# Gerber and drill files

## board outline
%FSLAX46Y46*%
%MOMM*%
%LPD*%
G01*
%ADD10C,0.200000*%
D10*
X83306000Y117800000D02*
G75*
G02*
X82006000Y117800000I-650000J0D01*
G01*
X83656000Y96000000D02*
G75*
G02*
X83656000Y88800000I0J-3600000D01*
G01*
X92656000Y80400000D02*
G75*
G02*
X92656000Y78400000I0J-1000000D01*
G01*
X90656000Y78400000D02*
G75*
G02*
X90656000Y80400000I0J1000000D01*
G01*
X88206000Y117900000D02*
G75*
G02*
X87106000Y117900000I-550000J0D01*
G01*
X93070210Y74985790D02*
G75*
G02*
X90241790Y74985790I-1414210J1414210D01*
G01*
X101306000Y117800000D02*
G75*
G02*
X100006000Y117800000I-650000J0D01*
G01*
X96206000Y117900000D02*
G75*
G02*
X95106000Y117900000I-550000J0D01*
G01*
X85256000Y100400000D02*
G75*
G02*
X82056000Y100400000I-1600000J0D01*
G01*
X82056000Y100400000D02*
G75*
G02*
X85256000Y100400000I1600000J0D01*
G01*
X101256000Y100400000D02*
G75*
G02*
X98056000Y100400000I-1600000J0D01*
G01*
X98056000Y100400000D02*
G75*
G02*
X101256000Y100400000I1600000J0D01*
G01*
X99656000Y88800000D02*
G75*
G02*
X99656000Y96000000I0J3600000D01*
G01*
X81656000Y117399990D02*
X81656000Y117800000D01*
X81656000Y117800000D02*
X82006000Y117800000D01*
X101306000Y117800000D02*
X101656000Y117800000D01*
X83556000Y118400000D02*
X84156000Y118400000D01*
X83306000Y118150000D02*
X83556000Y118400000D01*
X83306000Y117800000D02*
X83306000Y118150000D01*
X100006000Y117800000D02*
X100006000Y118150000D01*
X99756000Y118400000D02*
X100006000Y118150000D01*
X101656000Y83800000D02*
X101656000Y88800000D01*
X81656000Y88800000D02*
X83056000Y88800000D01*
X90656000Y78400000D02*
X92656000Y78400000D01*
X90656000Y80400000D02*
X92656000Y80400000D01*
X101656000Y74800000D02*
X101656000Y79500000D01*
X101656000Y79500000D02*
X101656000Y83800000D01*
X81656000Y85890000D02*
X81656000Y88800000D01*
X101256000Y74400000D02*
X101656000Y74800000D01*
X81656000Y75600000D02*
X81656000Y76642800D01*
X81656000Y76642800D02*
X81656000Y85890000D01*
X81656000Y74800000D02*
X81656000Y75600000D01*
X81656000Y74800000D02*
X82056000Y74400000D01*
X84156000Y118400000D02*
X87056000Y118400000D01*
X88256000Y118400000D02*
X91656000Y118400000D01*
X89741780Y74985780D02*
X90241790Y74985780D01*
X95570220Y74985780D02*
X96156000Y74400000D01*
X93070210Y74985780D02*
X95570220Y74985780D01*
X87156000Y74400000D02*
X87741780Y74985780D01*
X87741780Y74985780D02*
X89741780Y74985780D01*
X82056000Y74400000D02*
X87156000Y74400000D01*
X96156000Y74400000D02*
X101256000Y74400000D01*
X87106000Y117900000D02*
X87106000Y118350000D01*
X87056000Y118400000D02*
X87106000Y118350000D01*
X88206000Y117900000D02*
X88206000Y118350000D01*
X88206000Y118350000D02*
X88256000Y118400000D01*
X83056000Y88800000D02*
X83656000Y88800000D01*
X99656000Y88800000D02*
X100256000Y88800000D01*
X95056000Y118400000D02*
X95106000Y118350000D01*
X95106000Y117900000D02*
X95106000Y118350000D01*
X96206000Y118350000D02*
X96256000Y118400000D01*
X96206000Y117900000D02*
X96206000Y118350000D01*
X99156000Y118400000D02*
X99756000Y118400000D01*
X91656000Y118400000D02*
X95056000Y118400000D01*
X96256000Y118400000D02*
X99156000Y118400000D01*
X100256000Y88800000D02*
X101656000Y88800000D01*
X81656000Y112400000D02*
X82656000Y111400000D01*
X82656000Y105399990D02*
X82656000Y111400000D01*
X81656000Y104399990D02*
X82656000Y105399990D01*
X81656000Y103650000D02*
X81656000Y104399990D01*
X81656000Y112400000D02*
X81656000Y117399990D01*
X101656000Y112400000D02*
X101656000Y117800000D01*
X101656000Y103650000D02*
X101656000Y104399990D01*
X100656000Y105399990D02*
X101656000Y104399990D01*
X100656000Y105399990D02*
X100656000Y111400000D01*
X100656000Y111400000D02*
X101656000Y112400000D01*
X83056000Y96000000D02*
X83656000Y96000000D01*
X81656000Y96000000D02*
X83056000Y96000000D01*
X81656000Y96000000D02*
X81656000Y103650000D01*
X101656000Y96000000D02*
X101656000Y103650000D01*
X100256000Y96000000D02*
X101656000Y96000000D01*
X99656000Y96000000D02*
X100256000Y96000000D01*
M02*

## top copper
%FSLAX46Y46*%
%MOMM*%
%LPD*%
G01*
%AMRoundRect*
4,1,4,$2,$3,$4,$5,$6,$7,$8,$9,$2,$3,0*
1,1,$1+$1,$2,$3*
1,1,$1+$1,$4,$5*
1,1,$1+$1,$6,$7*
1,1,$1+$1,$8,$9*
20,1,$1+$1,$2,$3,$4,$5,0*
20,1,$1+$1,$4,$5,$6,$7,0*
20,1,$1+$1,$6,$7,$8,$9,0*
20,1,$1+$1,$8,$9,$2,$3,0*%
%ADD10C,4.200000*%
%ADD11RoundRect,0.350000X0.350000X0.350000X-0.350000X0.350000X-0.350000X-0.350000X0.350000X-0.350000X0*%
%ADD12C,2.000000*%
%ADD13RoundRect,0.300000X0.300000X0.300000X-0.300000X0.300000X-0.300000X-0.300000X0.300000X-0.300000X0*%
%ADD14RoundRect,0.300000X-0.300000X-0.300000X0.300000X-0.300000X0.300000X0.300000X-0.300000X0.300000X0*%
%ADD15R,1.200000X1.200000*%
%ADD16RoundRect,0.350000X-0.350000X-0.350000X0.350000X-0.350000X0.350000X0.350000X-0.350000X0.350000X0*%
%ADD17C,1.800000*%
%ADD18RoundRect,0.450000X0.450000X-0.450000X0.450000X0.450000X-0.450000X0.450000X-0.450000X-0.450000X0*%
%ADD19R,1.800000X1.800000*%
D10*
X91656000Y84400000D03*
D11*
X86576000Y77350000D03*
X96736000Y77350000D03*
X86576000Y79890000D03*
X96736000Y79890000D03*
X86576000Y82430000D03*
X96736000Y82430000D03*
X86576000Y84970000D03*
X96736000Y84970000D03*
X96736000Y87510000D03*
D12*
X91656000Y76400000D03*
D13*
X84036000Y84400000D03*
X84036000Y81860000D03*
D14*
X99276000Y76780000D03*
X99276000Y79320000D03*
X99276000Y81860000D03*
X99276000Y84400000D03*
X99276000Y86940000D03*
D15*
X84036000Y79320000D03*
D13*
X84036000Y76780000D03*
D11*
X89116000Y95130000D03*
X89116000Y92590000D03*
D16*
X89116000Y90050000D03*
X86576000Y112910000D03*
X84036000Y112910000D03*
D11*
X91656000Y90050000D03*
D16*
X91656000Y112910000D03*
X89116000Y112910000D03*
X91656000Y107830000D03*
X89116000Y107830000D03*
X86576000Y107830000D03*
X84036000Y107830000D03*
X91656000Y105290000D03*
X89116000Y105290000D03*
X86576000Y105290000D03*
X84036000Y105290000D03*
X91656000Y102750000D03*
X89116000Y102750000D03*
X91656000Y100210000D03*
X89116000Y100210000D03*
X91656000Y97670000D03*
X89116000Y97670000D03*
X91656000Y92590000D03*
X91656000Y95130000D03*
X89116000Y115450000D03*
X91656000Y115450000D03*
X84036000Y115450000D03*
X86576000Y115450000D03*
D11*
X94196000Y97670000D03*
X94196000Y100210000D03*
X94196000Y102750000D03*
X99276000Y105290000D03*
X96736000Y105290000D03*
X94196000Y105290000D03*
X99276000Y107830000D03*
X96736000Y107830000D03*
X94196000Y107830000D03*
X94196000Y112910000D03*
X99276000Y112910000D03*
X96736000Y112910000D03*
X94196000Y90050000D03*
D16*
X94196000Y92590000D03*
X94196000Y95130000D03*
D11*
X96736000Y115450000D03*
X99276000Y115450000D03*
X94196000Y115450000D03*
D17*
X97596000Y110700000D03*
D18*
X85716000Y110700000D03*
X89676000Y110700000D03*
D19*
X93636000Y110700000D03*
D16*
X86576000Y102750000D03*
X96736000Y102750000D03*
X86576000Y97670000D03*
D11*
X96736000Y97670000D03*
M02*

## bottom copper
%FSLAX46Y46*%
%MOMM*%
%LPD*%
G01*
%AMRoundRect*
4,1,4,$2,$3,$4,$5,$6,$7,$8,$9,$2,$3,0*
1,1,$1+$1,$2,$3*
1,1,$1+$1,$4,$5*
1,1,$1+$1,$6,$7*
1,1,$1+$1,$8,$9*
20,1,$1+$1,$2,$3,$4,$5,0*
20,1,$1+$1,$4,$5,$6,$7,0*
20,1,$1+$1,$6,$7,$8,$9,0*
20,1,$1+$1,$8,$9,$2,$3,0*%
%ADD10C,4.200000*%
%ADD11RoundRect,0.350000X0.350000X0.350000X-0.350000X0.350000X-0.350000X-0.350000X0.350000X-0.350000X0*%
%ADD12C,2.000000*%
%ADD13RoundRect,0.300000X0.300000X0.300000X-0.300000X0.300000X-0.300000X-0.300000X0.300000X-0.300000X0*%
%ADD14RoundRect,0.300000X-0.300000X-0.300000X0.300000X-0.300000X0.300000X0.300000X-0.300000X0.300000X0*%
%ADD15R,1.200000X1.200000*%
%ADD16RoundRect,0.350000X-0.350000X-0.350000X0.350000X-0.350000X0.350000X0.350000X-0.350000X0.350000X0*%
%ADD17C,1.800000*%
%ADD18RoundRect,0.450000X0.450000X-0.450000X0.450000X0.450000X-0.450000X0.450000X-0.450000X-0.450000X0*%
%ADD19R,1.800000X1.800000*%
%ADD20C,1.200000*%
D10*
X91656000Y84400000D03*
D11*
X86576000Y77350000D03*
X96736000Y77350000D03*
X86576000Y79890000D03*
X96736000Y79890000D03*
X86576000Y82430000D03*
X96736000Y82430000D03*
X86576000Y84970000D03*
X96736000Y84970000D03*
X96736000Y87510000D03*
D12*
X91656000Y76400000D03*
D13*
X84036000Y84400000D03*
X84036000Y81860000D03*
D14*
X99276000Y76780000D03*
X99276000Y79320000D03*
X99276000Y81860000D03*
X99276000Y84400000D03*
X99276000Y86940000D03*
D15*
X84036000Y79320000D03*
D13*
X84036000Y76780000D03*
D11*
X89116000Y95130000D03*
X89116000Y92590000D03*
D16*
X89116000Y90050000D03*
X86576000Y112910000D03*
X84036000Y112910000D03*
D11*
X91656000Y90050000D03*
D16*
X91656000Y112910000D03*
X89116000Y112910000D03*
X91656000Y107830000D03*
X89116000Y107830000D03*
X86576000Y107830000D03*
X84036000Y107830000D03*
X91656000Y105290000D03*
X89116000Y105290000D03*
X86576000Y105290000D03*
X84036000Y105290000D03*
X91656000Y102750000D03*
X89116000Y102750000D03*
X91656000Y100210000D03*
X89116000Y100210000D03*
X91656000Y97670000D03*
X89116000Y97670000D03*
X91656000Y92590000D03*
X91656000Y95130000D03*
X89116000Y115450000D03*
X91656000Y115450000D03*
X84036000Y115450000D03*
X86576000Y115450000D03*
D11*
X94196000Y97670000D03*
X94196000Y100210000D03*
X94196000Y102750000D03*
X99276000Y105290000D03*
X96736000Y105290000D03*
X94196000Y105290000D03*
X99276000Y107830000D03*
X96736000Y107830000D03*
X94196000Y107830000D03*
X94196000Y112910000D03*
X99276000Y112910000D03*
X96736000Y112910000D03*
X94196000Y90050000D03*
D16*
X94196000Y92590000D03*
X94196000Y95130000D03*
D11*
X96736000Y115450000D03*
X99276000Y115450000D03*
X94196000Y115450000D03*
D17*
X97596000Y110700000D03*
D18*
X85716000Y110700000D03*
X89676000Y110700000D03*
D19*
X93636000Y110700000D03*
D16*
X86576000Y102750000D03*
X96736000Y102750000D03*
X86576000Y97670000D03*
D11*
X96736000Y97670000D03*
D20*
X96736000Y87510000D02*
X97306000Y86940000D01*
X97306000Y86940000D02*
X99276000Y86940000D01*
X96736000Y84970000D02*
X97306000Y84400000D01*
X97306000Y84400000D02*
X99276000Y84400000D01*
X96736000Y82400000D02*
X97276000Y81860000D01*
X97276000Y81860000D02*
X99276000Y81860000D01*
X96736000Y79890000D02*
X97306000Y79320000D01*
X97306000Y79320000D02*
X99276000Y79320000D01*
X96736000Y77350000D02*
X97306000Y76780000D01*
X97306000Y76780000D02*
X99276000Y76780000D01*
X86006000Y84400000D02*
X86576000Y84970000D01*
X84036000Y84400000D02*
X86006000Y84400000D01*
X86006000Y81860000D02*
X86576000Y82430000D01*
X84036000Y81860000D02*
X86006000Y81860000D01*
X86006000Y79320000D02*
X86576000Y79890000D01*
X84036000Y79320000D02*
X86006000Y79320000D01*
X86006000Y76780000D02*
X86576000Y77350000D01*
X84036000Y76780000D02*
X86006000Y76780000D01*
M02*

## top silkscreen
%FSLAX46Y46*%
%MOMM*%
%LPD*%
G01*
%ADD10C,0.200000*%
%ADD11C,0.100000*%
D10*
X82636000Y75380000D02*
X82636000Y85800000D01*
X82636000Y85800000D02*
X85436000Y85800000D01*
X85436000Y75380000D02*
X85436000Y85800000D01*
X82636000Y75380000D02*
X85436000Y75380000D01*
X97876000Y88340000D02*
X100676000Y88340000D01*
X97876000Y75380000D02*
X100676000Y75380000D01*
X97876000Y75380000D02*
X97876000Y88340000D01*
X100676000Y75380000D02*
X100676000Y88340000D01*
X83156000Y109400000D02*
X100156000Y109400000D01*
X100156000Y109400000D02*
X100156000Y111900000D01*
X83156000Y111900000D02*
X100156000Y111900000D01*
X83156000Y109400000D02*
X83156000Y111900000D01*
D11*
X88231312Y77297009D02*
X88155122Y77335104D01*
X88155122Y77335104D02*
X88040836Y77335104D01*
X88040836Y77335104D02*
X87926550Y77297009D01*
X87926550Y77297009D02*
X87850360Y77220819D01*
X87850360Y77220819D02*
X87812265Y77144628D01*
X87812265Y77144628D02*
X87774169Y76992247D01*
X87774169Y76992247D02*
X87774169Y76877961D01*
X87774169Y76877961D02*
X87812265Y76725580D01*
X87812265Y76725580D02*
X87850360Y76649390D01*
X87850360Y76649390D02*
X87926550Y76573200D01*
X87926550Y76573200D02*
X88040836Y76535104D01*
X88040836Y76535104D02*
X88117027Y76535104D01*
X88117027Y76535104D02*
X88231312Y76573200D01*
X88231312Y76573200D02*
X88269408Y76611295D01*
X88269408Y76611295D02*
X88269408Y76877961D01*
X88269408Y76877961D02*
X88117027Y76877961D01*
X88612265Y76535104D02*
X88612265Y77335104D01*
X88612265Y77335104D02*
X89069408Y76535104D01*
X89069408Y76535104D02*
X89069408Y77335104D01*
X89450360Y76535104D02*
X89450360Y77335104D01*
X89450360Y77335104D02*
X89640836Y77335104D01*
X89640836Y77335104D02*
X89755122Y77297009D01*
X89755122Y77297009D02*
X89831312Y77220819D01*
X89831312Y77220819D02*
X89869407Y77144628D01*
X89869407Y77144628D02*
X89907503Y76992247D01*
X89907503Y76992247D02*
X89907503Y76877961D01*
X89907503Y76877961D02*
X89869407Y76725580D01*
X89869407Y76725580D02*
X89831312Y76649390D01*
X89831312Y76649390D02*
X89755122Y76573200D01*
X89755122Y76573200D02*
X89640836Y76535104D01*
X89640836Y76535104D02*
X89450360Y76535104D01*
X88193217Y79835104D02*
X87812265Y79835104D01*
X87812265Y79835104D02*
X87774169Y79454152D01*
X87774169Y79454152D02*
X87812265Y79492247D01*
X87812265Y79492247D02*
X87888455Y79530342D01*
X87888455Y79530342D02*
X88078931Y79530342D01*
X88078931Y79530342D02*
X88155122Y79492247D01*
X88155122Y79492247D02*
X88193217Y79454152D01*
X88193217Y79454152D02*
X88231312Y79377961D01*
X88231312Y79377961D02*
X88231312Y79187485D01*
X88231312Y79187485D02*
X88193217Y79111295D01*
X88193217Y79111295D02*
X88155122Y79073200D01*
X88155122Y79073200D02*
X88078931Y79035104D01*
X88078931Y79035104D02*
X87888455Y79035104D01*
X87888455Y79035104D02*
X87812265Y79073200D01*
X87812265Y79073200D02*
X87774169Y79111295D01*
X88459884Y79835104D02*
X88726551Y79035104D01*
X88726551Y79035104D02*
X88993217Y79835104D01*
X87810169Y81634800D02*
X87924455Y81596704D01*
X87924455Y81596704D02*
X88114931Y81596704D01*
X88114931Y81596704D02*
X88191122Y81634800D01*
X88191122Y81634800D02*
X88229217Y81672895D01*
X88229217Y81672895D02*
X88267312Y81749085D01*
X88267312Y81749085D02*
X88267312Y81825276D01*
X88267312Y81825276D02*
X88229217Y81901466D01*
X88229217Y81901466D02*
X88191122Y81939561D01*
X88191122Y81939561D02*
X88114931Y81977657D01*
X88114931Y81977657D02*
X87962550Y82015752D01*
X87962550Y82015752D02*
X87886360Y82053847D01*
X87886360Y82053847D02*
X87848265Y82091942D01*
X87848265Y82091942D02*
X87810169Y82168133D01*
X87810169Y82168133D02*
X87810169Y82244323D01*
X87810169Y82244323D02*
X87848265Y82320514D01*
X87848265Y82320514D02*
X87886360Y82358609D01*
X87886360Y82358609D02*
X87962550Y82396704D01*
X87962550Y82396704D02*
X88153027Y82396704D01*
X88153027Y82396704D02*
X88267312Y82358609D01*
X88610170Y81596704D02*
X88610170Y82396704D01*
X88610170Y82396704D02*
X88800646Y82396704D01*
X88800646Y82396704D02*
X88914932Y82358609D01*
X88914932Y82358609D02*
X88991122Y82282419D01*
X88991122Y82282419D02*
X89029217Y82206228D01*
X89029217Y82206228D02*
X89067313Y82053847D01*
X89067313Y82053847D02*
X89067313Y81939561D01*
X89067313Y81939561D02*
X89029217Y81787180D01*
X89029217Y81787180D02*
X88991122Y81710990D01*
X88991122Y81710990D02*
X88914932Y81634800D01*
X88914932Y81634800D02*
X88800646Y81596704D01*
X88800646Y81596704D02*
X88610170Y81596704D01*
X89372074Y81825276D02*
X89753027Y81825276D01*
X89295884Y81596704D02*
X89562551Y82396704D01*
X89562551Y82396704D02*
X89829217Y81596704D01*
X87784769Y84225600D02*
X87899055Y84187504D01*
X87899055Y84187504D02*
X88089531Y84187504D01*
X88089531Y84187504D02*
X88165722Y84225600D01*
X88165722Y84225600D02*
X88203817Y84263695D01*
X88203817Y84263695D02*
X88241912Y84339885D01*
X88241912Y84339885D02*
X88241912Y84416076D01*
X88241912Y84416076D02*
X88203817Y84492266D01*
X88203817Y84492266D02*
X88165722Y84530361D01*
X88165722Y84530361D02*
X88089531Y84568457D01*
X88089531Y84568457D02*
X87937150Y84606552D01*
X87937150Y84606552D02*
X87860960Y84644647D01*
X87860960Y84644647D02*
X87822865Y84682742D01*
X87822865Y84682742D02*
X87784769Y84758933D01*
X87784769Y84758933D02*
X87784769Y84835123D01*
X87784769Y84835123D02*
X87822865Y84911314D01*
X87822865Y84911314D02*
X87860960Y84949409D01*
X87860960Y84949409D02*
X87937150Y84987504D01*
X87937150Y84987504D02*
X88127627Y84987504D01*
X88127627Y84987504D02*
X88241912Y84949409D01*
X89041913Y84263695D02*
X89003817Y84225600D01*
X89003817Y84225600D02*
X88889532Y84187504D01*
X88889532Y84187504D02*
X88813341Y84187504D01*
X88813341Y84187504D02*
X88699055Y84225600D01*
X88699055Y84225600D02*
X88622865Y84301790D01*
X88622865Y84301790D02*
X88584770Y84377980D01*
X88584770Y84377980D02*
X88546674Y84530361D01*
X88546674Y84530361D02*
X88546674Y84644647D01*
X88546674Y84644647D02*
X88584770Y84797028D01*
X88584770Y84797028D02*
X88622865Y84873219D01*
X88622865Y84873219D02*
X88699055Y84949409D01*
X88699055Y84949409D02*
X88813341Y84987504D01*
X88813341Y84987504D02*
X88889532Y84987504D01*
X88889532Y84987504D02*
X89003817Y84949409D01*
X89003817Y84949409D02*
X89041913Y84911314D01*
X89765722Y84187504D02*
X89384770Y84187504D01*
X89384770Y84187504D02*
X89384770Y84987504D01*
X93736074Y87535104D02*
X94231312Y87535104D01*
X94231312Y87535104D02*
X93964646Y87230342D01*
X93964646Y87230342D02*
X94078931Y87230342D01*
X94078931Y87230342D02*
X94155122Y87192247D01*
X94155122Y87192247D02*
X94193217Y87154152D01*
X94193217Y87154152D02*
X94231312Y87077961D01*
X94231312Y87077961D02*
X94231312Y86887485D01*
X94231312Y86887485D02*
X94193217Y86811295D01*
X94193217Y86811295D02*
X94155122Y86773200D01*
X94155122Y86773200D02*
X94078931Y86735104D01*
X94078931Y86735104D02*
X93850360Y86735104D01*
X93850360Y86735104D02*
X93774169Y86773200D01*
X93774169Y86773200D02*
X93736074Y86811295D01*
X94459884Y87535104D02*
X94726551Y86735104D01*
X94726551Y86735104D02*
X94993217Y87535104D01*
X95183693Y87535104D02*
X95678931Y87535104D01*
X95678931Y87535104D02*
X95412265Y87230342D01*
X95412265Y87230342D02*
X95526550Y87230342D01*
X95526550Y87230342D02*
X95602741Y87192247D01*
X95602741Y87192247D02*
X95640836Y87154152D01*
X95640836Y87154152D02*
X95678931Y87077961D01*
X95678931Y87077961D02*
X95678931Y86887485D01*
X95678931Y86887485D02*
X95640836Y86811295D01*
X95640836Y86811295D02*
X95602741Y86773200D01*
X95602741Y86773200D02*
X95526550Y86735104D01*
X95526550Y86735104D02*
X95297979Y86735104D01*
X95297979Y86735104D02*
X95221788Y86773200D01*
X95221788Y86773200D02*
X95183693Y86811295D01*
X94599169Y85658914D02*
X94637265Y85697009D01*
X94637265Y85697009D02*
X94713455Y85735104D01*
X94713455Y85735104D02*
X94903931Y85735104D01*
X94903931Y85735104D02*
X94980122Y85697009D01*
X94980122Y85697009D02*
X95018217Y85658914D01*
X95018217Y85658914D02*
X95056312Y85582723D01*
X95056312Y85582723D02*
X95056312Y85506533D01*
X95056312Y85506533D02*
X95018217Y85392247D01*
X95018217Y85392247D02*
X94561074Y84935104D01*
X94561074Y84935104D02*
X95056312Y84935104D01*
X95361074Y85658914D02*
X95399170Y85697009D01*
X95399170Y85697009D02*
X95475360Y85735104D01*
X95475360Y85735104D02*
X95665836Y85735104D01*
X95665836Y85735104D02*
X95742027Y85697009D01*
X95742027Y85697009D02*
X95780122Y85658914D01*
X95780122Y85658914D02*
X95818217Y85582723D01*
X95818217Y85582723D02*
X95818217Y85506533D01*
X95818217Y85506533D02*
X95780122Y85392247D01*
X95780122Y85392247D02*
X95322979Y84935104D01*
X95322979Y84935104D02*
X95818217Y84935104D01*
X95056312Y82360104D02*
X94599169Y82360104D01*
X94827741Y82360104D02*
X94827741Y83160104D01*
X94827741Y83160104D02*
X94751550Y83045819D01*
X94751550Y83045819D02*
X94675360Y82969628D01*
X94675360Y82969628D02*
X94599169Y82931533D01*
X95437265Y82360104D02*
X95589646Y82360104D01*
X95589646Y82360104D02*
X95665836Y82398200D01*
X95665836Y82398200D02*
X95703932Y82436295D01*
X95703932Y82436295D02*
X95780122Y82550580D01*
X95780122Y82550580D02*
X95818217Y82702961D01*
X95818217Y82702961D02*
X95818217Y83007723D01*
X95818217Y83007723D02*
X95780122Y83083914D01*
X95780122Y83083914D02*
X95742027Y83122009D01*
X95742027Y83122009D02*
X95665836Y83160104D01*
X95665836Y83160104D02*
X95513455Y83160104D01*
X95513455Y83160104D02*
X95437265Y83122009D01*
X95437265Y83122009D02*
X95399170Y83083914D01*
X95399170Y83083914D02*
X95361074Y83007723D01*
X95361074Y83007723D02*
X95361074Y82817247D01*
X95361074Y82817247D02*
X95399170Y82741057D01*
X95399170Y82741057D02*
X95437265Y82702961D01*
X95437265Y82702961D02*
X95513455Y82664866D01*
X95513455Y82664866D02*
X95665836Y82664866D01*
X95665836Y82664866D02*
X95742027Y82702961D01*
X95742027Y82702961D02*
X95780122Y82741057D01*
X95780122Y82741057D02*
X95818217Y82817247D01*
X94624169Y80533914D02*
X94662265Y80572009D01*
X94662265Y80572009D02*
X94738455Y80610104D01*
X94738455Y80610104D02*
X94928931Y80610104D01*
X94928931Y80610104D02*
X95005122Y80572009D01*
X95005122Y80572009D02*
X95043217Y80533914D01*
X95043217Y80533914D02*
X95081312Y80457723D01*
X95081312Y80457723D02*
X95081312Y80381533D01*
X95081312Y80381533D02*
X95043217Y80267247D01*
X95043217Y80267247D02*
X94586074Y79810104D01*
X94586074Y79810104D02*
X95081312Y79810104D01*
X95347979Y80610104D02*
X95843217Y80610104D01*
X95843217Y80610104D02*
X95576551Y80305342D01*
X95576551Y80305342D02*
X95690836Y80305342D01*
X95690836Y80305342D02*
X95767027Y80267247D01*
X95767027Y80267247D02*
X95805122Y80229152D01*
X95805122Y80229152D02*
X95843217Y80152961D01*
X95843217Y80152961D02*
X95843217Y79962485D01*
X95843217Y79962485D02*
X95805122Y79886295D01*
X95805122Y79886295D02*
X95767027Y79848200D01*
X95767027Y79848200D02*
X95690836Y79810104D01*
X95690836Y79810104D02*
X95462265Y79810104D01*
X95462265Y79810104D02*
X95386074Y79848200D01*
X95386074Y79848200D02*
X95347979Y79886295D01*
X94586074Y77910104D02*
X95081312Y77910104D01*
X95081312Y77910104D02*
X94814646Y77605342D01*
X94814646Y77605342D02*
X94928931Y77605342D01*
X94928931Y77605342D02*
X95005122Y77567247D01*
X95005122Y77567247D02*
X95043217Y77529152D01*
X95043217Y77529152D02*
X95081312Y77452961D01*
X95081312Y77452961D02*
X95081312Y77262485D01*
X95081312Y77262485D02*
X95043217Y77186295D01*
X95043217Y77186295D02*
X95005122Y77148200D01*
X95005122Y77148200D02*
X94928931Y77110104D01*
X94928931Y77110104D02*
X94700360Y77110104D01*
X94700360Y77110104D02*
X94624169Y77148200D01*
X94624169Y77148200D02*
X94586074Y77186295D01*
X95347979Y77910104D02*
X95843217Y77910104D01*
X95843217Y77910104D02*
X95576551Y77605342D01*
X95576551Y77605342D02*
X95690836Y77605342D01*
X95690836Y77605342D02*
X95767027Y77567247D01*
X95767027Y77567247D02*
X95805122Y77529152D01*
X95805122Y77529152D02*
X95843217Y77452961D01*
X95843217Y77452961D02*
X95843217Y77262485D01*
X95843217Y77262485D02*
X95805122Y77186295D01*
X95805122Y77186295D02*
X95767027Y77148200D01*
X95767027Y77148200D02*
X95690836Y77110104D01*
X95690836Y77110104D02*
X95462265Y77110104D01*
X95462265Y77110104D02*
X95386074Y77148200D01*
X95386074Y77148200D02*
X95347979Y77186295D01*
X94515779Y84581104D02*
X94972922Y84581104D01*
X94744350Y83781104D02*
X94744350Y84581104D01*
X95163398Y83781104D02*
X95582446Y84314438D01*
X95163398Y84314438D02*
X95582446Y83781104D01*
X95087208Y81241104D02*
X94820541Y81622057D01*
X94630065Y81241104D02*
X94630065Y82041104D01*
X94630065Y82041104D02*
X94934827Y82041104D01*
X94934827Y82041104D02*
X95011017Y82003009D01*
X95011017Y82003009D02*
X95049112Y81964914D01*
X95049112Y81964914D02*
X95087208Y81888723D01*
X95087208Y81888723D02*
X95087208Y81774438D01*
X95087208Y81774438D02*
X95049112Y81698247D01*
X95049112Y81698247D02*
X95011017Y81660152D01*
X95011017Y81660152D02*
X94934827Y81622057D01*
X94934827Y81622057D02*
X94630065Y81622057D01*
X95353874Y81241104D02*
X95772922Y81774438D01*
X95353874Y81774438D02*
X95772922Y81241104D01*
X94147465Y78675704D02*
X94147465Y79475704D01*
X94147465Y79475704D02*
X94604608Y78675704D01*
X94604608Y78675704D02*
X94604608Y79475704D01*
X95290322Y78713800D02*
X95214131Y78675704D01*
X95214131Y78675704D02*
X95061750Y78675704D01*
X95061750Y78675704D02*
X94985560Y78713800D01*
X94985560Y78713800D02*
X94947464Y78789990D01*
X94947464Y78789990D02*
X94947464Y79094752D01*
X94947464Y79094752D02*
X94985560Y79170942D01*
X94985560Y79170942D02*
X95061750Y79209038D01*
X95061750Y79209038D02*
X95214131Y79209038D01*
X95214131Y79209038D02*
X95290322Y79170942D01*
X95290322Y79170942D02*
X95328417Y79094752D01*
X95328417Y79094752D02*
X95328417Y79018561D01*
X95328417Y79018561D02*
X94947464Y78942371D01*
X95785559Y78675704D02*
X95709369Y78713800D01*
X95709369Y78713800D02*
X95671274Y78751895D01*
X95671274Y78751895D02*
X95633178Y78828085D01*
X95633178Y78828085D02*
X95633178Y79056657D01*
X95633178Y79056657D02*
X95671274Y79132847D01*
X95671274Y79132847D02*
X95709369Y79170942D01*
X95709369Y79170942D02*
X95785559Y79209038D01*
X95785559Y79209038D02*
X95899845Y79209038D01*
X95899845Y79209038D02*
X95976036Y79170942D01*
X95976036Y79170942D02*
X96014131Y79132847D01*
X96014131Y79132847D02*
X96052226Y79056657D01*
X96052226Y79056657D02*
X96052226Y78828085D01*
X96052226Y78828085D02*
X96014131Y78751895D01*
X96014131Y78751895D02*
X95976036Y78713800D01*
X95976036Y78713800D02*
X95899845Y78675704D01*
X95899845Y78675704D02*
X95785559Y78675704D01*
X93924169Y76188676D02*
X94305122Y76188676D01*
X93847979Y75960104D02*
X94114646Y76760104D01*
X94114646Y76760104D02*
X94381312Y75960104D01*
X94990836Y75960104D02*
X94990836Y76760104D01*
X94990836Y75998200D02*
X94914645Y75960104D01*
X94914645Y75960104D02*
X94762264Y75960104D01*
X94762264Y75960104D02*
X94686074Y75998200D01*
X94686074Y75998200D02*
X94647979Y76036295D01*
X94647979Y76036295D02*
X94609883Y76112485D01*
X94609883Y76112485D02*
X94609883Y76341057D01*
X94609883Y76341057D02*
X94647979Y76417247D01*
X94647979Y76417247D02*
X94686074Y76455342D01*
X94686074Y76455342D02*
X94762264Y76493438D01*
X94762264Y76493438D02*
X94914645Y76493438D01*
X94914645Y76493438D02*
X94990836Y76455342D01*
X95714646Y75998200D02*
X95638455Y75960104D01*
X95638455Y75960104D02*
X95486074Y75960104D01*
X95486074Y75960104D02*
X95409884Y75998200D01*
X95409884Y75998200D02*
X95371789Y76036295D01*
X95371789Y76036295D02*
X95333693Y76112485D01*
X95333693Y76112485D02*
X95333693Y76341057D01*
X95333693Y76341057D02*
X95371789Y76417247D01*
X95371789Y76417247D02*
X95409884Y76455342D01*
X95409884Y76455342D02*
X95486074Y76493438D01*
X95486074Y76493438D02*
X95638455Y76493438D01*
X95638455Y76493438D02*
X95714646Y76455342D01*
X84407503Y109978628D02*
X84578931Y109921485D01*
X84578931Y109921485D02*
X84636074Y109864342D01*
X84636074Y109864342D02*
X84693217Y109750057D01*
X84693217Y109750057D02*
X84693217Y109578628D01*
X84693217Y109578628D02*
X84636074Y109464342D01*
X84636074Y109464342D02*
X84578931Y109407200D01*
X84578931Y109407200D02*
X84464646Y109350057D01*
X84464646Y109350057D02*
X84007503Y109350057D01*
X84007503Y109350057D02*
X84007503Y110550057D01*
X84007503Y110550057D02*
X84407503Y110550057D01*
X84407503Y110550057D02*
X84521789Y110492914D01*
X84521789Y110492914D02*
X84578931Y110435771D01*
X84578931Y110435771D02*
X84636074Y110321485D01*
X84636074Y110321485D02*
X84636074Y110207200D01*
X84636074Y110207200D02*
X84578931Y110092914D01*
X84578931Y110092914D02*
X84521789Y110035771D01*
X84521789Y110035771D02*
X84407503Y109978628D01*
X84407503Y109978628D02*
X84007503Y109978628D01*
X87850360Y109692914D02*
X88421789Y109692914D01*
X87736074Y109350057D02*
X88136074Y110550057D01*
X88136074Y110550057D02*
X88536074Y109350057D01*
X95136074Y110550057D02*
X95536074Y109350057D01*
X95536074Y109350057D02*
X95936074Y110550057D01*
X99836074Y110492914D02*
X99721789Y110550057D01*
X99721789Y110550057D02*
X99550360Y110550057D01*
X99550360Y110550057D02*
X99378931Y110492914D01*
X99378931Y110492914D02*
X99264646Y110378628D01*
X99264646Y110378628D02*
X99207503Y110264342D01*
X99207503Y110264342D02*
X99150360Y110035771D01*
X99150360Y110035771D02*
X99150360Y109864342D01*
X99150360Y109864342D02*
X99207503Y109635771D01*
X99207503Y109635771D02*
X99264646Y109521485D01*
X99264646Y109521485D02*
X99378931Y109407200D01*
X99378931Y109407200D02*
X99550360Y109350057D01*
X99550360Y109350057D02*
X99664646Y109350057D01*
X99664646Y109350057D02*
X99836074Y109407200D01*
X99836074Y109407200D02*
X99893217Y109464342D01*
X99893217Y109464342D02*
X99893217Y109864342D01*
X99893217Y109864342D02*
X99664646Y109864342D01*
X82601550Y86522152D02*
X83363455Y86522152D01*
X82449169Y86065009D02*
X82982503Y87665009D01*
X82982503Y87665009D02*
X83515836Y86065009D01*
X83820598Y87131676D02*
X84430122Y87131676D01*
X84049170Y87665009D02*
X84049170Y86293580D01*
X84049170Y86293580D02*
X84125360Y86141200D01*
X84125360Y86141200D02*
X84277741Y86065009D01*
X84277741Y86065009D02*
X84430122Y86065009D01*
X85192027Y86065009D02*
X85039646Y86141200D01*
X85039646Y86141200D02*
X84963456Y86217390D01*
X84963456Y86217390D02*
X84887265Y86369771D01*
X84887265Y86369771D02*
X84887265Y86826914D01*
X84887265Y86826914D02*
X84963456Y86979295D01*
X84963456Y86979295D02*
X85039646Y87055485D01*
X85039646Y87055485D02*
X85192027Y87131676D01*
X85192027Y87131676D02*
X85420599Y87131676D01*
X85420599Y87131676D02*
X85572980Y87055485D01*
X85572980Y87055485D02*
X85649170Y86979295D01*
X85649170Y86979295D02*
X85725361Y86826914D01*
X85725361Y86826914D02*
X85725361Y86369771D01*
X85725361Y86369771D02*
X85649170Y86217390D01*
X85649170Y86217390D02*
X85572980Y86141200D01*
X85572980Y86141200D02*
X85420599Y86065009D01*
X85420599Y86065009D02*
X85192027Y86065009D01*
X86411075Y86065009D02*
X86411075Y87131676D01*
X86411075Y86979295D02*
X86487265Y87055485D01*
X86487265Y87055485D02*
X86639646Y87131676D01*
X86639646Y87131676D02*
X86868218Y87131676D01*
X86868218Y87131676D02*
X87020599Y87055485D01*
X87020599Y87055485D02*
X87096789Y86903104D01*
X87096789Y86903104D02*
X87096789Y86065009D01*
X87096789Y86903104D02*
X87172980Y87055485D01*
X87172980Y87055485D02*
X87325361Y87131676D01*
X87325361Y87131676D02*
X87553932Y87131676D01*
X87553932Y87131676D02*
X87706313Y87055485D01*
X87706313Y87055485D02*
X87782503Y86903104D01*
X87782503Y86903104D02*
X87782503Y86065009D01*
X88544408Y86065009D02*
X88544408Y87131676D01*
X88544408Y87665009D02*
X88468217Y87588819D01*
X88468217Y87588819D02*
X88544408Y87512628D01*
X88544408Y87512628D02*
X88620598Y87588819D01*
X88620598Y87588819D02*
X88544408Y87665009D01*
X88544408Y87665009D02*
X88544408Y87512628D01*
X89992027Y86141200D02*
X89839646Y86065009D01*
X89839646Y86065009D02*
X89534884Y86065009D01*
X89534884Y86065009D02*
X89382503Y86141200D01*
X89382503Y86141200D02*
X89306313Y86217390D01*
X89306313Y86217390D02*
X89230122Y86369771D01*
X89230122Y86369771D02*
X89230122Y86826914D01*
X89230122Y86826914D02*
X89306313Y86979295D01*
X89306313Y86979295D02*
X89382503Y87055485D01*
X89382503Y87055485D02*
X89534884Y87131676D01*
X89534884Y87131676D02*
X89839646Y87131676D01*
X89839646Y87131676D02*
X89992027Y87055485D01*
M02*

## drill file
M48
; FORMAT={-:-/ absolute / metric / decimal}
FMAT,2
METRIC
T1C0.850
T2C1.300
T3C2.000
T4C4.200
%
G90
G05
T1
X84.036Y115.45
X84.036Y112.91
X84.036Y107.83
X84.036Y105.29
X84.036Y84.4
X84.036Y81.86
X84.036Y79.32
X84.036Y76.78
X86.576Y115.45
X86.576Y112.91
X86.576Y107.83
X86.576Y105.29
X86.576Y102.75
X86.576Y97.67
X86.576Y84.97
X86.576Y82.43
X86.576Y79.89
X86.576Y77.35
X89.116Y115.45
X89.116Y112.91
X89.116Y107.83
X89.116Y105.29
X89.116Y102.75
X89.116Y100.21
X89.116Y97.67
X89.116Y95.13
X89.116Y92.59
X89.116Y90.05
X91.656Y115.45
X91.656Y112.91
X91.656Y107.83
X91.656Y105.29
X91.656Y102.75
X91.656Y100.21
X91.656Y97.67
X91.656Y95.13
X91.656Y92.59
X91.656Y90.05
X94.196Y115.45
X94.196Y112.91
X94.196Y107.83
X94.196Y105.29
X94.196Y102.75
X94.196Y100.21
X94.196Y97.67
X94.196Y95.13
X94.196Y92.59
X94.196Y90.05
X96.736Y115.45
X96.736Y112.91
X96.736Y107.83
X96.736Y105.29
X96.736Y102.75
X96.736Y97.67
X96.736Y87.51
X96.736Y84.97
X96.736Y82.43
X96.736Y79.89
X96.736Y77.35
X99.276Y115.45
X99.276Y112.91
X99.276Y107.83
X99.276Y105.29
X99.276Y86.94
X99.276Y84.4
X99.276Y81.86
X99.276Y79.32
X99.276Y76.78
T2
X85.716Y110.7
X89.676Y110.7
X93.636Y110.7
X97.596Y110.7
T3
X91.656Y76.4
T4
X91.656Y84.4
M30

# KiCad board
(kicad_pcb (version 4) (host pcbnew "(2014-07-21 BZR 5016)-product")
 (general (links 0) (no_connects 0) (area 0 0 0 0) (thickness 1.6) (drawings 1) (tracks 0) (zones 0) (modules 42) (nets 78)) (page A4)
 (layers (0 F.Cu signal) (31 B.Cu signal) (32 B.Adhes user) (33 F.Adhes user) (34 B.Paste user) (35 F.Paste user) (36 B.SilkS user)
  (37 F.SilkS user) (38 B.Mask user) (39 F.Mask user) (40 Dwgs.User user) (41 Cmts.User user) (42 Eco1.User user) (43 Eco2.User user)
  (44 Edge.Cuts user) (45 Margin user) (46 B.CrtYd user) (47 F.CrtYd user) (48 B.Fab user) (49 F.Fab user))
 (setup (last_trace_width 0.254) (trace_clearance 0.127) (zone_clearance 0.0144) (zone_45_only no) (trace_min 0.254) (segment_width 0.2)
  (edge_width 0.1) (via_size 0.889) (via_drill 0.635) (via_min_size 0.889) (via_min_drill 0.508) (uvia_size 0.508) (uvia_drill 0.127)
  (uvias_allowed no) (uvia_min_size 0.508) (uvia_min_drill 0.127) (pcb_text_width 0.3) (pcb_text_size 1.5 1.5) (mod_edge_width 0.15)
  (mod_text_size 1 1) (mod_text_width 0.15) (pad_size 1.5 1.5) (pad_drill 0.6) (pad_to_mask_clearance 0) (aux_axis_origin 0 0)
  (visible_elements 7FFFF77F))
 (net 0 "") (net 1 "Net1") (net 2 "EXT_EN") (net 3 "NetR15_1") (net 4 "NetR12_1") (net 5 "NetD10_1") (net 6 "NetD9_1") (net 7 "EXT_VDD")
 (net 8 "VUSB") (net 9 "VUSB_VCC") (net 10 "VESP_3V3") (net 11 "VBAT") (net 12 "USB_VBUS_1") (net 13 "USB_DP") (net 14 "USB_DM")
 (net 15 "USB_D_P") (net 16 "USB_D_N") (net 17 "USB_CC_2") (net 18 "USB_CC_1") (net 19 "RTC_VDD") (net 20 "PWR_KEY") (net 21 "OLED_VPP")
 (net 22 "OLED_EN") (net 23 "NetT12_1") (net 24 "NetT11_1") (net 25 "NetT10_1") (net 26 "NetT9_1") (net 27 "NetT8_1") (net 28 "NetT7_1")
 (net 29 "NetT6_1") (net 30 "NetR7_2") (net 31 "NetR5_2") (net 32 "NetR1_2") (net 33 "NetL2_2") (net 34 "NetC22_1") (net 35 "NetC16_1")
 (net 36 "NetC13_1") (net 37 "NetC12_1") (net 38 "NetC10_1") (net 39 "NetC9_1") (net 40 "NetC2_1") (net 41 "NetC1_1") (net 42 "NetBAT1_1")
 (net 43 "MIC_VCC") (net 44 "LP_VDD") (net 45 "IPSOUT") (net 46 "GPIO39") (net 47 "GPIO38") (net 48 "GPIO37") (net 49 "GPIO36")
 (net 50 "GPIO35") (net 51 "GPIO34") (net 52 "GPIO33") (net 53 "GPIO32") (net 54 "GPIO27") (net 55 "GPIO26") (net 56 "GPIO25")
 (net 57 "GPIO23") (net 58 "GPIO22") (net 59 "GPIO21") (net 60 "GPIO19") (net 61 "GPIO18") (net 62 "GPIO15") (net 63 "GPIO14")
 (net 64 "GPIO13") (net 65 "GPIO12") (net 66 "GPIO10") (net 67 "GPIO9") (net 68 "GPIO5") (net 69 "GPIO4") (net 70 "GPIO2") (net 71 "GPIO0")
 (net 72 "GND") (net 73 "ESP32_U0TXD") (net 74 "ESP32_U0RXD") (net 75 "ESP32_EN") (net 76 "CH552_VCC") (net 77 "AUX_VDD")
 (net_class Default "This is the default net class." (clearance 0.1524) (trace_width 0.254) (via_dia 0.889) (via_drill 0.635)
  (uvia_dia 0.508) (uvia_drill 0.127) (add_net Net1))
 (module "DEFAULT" (layer F.Cu) (at 0 0)
  (pad "" thru_hole circle (at 91.65600 -84.40000) (size 4.2 4.2) (drill 4.2) (layers *.Cu))
  (pad "" thru_hole roundrect (at 86.57600 -77.35000 180) (size 1.4 1.4) (drill 0.85) (roundrect_rratio 0.25) (layers *.Cu))
  (pad "" thru_hole roundrect (at 96.73600 -77.35000 180) (size 1.4 1.4) (drill 0.85) (roundrect_rratio 0.25) (layers *.Cu))
  (pad "" thru_hole roundrect (at 86.57600 -79.89000 180) (size 1.4 1.4) (drill 0.85) (roundrect_rratio 0.25) (layers *.Cu))
  (pad "" thru_hole roundrect (at 96.73600 -79.89000 180) (size 1.4 1.4) (drill 0.85) (roundrect_rratio 0.25) (layers *.Cu))
  (pad "" thru_hole roundrect (at 86.57600 -82.43000 180) (size 1.4 1.4) (drill 0.85) (roundrect_rratio 0.25) (layers *.Cu))
  (pad "" thru_hole roundrect (at 96.73600 -82.43000 180) (size 1.4 1.4) (drill 0.85) (roundrect_rratio 0.25) (layers *.Cu))
  (pad "" thru_hole roundrect (at 86.57600 -84.97000 180) (size 1.4 1.4) (drill 0.85) (roundrect_rratio 0.25) (layers *.Cu))
  (pad "" thru_hole roundrect (at 96.73600 -84.97000 180) (size 1.4 1.4) (drill 0.85) (roundrect_rratio 0.25) (layers *.Cu))
  (pad "" thru_hole roundrect (at 96.73600 -87.51000 180) (size 1.4 1.4) (drill 0.85) (roundrect_rratio 0.25) (layers *.Cu))
  (pad "" thru_hole circle (at 91.65600 -76.40000) (size 2 2) (drill 2) (layers *.Cu))
  (pad "SCLG22" thru_hole roundrect (at 84.03600 -84.40000 180) (size 1.2 1.2) (drill 0.85) (roundrect_rratio 0.25) (layers *.Cu))
  (pad "SDAG21" thru_hole roundrect (at 84.03600 -81.86000 180) (size 1.2 1.2) (drill 0.85) (roundrect_rratio 0.25) (layers *.Cu))
  (pad "" thru_hole roundrect (at 99.27600 -76.78000) (size 1.2 1.2) (drill 0.85) (roundrect_rratio 0.25) (layers *.Cu))
  (pad "" thru_hole roundrect (at 99.27600 -79.32000) (size 1.2 1.2) (drill 0.85) (roundrect_rratio 0.25) (layers *.Cu))
  (pad "" thru_hole roundrect (at 99.27600 -81.86000) (size 1.2 1.2) (drill 0.85) (roundrect_rratio 0.25) (layers *.Cu))
  (pad "" thru_hole roundrect (at 99.27600 -84.40000) (size 1.2 1.2) (drill 0.85) (roundrect_rratio 0.25) (layers *.Cu))
  (pad "3V3" thru_hole roundrect (at 99.27600 -86.94000) (size 1.2 1.2) (drill 0.85) (roundrect_rratio 0.25) (layers *.Cu))
  (pad "5V" thru_hole rect (at 84.03600 -79.32000 180) (size 1.2 1.2) (drill 0.85) (layers *.Cu))
  (pad "GND" thru_hole roundrect (at 84.03600 -76.78000 180) (size 1.2 1.2) (drill 0.85) (roundrect_rratio 0.25) (layers *.Cu))
  (pad "" thru_hole roundrect (at 89.11600 -95.13000 180) (size 1.4 1.4) (drill 0.85) (roundrect_rratio 0.25) (layers *.Cu))
  (pad "" thru_hole roundrect (at 89.11600 -92.59000 180) (size 1.4 1.4) (drill 0.85) (roundrect_rratio 0.25) (layers *.Cu))
  (pad "" thru_hole roundrect (at 89.11600 -90.05000) (size 1.4 1.4) (drill 0.85) (roundrect_rratio 0.25) (layers *.Cu))
  (pad "" thru_hole roundrect (at 86.57600 -112.91000) (size 1.4 1.4) (drill 0.85) (roundrect_rratio 0.25) (layers *.Cu))
  (pad "" thru_hole roundrect (at 84.03600 -112.91000) (size 1.4 1.4) (drill 0.85) (roundrect_rratio 0.25) (layers *.Cu))
  (pad "" thru_hole roundrect (at 91.65600 -90.05000 180) (size 1.4 1.4) (drill 0.85) (roundrect_rratio 0.25) (layers *.Cu))
  (pad "" thru_hole roundrect (at 91.65600 -112.91000) (size 1.4 1.4) (drill 0.85) (roundrect_rratio 0.25) (layers *.Cu))
  (pad "" thru_hole roundrect (at 89.11600 -112.91000) (size 1.4 1.4) (drill 0.85) (roundrect_rratio 0.25) (layers *.Cu))
  (pad "" thru_hole roundrect (at 91.65600 -107.83000) (size 1.4 1.4) (drill 0.85) (roundrect_rratio 0.25) (layers *.Cu))
  (pad "" thru_hole roundrect (at 89.11600 -107.83000) (size 1.4 1.4) (drill 0.85) (roundrect_rratio 0.25) (layers *.Cu))
  (pad "" thru_hole roundrect (at 86.57600 -107.83000) (size 1.4 1.4) (drill 0.85) (roundrect_rratio 0.25) (layers *.Cu))
  (pad "" thru_hole roundrect (at 84.03600 -107.83000) (size 1.4 1.4) (drill 0.85) (roundrect_rratio 0.25) (layers *.Cu))
  (pad "" thru_hole roundrect (at 91.65600 -105.29000) (size 1.4 1.4) (drill 0.85) (roundrect_rratio 0.25) (layers *.Cu))
  (pad "" thru_hole roundrect (at 89.11600 -105.29000) (size 1.4 1.4) (drill 0.85) (roundrect_rratio 0.25) (layers *.Cu))
  (pad "" thru_hole roundrect (at 86.57600 -105.29000) (size 1.4 1.4) (drill 0.85) (roundrect_rratio 0.25) (layers *.Cu))
  (pad "" thru_hole roundrect (at 84.03600 -105.29000) (size 1.4 1.4) (drill 0.85) (roundrect_rratio 0.25) (layers *.Cu))
  (pad "" thru_hole roundrect (at 91.65600 -102.75000) (size 1.4 1.4) (drill 0.85) (roundrect_rratio 0.25) (layers *.Cu))
  (pad "" thru_hole roundrect (at 89.11600 -102.75000) (size 1.4 1.4) (drill 0.85) (roundrect_rratio 0.25) (layers *.Cu))
  (pad "" thru_hole roundrect (at 91.65600 -100.21000) (size 1.4 1.4) (drill 0.85) (roundrect_rratio 0.25) (layers *.Cu))
  (pad "" thru_hole roundrect (at 89.11600 -100.21000) (size 1.4 1.4) (drill 0.85) (roundrect_rratio 0.25) (layers *.Cu))
  (pad "" thru_hole roundrect (at 91.65600 -97.67000) (size 1.4 1.4) (drill 0.85) (roundrect_rratio 0.25) (layers *.Cu))
  (pad "" thru_hole roundrect (at 89.11600 -97.67000) (size 1.4 1.4) (drill 0.85) (roundrect_rratio 0.25) (layers *.Cu))
  (pad "" thru_hole roundrect (at 91.65600 -92.59000) (size 1.4 1.4) (drill 0.85) (roundrect_rratio 0.25) (layers *.Cu))
  (pad "" thru_hole roundrect (at 91.65600 -95.13000) (size 1.4 1.4) (drill 0.85) (roundrect_rratio 0.25) (layers *.Cu))
  (pad "" thru_hole roundrect (at 89.11600 -115.45000) (size 1.4 1.4) (drill 0.85) (roundrect_rratio 0.25) (layers *.Cu))
  (pad "" thru_hole roundrect (at 91.65600 -115.45000) (size 1.4 1.4) (drill 0.85) (roundrect_rratio 0.25) (layers *.Cu))
  (pad "" thru_hole roundrect (at 84.03600 -115.45000) (size 1.4 1.4) (drill 0.85) (roundrect_rratio 0.25) (layers *.Cu))
  (pad "" thru_hole roundrect (at 86.57600 -115.45000) (size 1.4 1.4) (drill 0.85) (roundrect_rratio 0.25) (layers *.Cu))
  (pad "" thru_hole roundrect (at 94.19600 -97.67000 180) (size 1.4 1.4) (drill 0.85) (roundrect_rratio 0.25) (layers *.Cu))
  (pad "" thru_hole roundrect (at 94.19600 -100.21000 180) (size 1.4 1.4) (drill 0.85) (roundrect_rratio 0.25) (layers *.Cu))
  (pad "" thru_hole roundrect (at 94.19600 -102.75000 180) (size 1.4 1.4) (drill 0.85) (roundrect_rratio 0.25) (layers *.Cu))
  (pad "" thru_hole roundrect (at 99.27600 -105.29000 180) (size 1.4 1.4) (drill 0.85) (roundrect_rratio 0.25) (layers *.Cu))
  (pad "" thru_hole roundrect (at 96.73600 -105.29000 180) (size 1.4 1.4) (drill 0.85) (roundrect_rratio 0.25) (layers *.Cu))
  (pad "" thru_hole roundrect (at 94.19600 -105.29000 180) (size 1.4 1.4) (drill 0.85) (roundrect_rratio 0.25) (layers *.Cu))
  (pad "" thru_hole roundrect (at 99.27600 -107.83000 180) (size 1.4 1.4) (drill 0.85) (roundrect_rratio 0.25) (layers *.Cu))
  (pad "" thru_hole roundrect (at 96.73600 -107.83000 180) (size 1.4 1.4) (drill 0.85) (roundrect_rratio 0.25) (layers *.Cu))
  (pad "" thru_hole roundrect (at 94.19600 -107.83000 180) (size 1.4 1.4) (drill 0.85) (roundrect_rratio 0.25) (layers *.Cu))
  (pad "" thru_hole roundrect (at 94.19600 -112.91000 180) (size 1.4 1.4) (drill 0.85) (roundrect_rratio 0.25) (layers *.Cu))
  (pad "" thru_hole roundrect (at 99.27600 -112.91000 180) (size 1.4 1.4) (drill 0.85) (roundrect_rratio 0.25) (layers *.Cu))
  (pad "" thru_hole roundrect (at 96.73600 -112.91000 180) (size 1.4 1.4) (drill 0.85) (roundrect_rratio 0.25) (layers *.Cu))
  (pad "" thru_hole roundrect (at 94.19600 -90.05000 180) (size 1.4 1.4) (drill 0.85) (roundrect_rratio 0.25) (layers *.Cu))
  (pad "" thru_hole roundrect (at 94.19600 -92.59000) (size 1.4 1.4) (drill 0.85) (roundrect_rratio 0.25) (layers *.Cu))
  (pad "" thru_hole roundrect (at 94.19600 -95.13000) (size 1.4 1.4) (drill 0.85) (roundrect_rratio 0.25) (layers *.Cu))
  (pad "" thru_hole roundrect (at 96.73600 -115.45000 180) (size 1.4 1.4) (drill 0.85) (roundrect_rratio 0.25) (layers *.Cu))
  (pad "" thru_hole roundrect (at 99.27600 -115.45000 180) (size 1.4 1.4) (drill 0.85) (roundrect_rratio 0.25) (layers *.Cu))
  (pad "" thru_hole roundrect (at 94.19600 -115.45000 180) (size 1.4 1.4) (drill 0.85) (roundrect_rratio 0.25) (layers *.Cu))
  (pad "G" thru_hole circle (at 97.59600 -110.70000 90) (size 1.8 1.8) (drill 1.3) (layers *.Cu))
  (pad "B" thru_hole roundrect (at 85.71600 -110.70000 90) (size 1.8 1.8) (drill 1.3) (roundrect_rratio 0.25) (layers *.Cu))
  (pad "A" thru_hole roundrect (at 89.67600 -110.70000 90) (size 1.8 1.8) (drill 1.3) (roundrect_rratio 0.25) (layers *.Cu))
  (pad "12V" thru_hole rect (at 93.63600 -110.70000 90) (size 1.8 1.8) (drill 1.3) (layers *.Cu))
  (pad "" thru_hole roundrect (at 86.57600 -102.75000) (size 1.4 1.4) (drill 0.85) (roundrect_rratio 0.25) (layers *.Cu))
  (pad "" thru_hole roundrect (at 96.73600 -102.75000) (size 1.4 1.4) (drill 0.85) (roundrect_rratio 0.25) (layers *.Cu))
  (pad "" thru_hole roundrect (at 86.57600 -97.67000) (size 1.4 1.4) (drill 0.85) (roundrect_rratio 0.25) (layers *.Cu))
  (pad "" thru_hole roundrect (at 96.73600 -97.67000 180) (size 1.4 1.4) (drill 0.85) (roundrect_rratio 0.25) (layers *.Cu))
  (pad "35" smd circle (at 91.65600 -76.40000) (size 3.9 3.9) (layers F.Mask))
  (pad "35" smd circle (at 91.65600 -76.40000 180) (size 3.9 3.9) (layers B.Mask)))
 (gr_arc (start 82.65600 -117.80000) (end 82.00600 -117.80000) (angle -180) (layer Edge.Cuts) (width 0.2))
 (gr_arc (start 83.65600 -92.40000) (end 83.65600 -88.80000) (angle -180) (layer Edge.Cuts) (width 0.2))
 (gr_arc (start 92.65600 -79.40000) (end 92.65600 -78.40000) (angle -180) (layer Edge.Cuts) (width 0.2))
 (gr_arc (start 90.65600 -79.40000) (end 90.65600 -80.40000) (angle -180) (layer Edge.Cuts) (width 0.2))
 (gr_arc (start 87.65600 -117.90000) (end 87.10600 -117.90000) (angle -180) (layer Edge.Cuts) (width 0.2))
 (gr_arc (start 91.65600 -76.40000) (end 90.24179 -74.98579) (angle -90) (layer Edge.Cuts) (width 0.2))
 (gr_arc (start 100.65600 -117.80000) (end 100.00600 -117.80000) (angle -180) (layer Edge.Cuts) (width 0.2))
 (gr_arc (start 95.65600 -117.90000) (end 95.10600 -117.90000) (angle -180) (layer Edge.Cuts) (width 0.2))
 (gr_arc (start 83.65600 -100.40000) (end 85.25600 -100.40000) (angle -360) (layer Edge.Cuts) (width 0.2))
 (gr_arc (start 99.65600 -100.40000) (end 101.25600 -100.40000) (angle -360) (layer Edge.Cuts) (width 0.2))
 (gr_arc (start 99.65600 -92.40000) (end 99.65600 -96.00000) (angle -180) (layer Edge.Cuts) (width 0.2))
 (gr_line (start 82.63600 -75.38000) (end 82.63600 -85.80000) (layer F.SilkS) (width 0.2))
 (gr_line (start 82.63600 -85.80000) (end 85.43600 -85.80000) (layer F.SilkS) (width 0.2))
 (gr_line (start 85.43600 -75.38000) (end 85.43600 -85.80000) (layer F.SilkS) (width 0.2))
 (gr_line (start 82.63600 -75.38000) (end 85.43600 -75.38000) (layer F.SilkS) (width 0.2))
 (gr_line (start 97.87600 -88.34000) (end 100.67600 -88.34000) (layer F.SilkS) (width 0.2))
 (gr_line (start 97.87600 -75.38000) (end 100.67600 -75.38000) (layer F.SilkS) (width 0.2))
 (gr_line (start 97.87600 -75.38000) (end 97.87600 -88.34000) (layer F.SilkS) (width 0.2))
 (gr_line (start 100.67600 -75.38000) (end 100.67600 -88.34000) (layer F.SilkS) (width 0.2))
 (gr_line (start 83.15600 -109.40000) (end 100.15600 -109.40000) (layer F.SilkS) (width 0.2))
 (gr_line (start 100.15600 -109.40000) (end 100.15600 -111.90000) (layer F.SilkS) (width 0.2))
 (gr_line (start 83.15600 -111.90000) (end 100.15600 -111.90000) (layer F.SilkS) (width 0.2))
 (gr_line (start 83.15600 -109.40000) (end 83.15600 -111.90000) (layer F.SilkS) (width 0.2))
 (gr_line (start 81.65600 -117.39999) (end 81.65600 -117.80000) (layer Edge.Cuts) (width 0.2))
 (gr_line (start 81.65600 -117.80000) (end 82.00600 -117.80000) (layer Edge.Cuts) (width 0.2))
 (gr_line (start 101.30600 -117.80000) (end 101.65600 -117.80000) (layer Edge.Cuts) (width 0.2))
 (gr_line (start 83.55600 -118.40000) (end 84.15600 -118.40000) (layer Edge.Cuts) (width 0.2))
 (gr_line (start 83.30600 -118.15000) (end 83.55600 -118.40000) (layer Edge.Cuts) (width 0.2))
 (gr_line (start 83.30600 -117.80000) (end 83.30600 -118.15000) (layer Edge.Cuts) (width 0.2))
 (gr_line (start 100.00600 -117.80000) (end 100.00600 -118.15000) (layer Edge.Cuts) (width 0.2))
 (gr_line (start 99.75600 -118.40000) (end 100.00600 -118.15000) (layer Edge.Cuts) (width 0.2))
 (gr_line (start 101.65600 -83.80000) (end 101.65600 -88.80000) (layer Edge.Cuts) (width 0.2))
 (gr_line (start 81.65600 -88.80000) (end 83.05600 -88.80000) (layer Edge.Cuts) (width 0.2))
 (gr_line (start 90.65600 -78.40000) (end 92.65600 -78.40000) (layer Edge.Cuts) (width 0.2))
 (gr_line (start 90.65600 -80.40000) (end 92.65600 -80.40000) (layer Edge.Cuts) (width 0.2))
 (gr_line (start 101.65600 -74.80000) (end 101.65600 -79.50000) (layer Edge.Cuts) (width 0.2))
 (gr_line (start 101.65600 -79.50000) (end 101.65600 -83.80000) (layer Edge.Cuts) (width 0.2))
 (gr_line (start 81.65600 -85.89000) (end 81.65600 -88.80000) (layer Edge.Cuts) (width 0.2))
 (gr_line (start 101.25600 -74.40000) (end 101.65600 -74.80000) (layer Edge.Cuts) (width 0.2))
 (gr_line (start 81.65600 -75.60000) (end 81.65600 -76.64280) (layer Edge.Cuts) (width 0.2))
 (gr_line (start 81.65600 -76.64280) (end 81.65600 -85.89000) (layer Edge.Cuts) (width 0.2))
 (gr_line (start 81.65600 -74.80000) (end 81.65600 -75.60000) (layer Edge.Cuts) (width 0.2))
 (gr_line (start 81.65600 -74.80000) (end 82.05600 -74.40000) (layer Edge.Cuts) (width 0.2))
 (gr_line (start 84.15600 -118.40000) (end 87.05600 -118.40000) (layer Edge.Cuts) (width 0.2))
 (gr_line (start 88.25600 -118.40000) (end 91.65600 -118.40000) (layer Edge.Cuts) (width 0.2))
 (gr_line (start 89.74178 -74.98578) (end 90.24179 -74.98578) (layer Edge.Cuts) (width 0.2))
 (gr_line (start 95.57022 -74.98578) (end 96.15600 -74.40000) (layer Edge.Cuts) (width 0.2))
 (gr_line (start 93.07021 -74.98578) (end 95.57022 -74.98578) (layer Edge.Cuts) (width 0.2))
 (gr_line (start 87.15600 -74.40000) (end 87.74178 -74.98578) (layer Edge.Cuts) (width 0.2))
 (gr_line (start 87.74178 -74.98578) (end 89.74178 -74.98578) (layer Edge.Cuts) (width 0.2))
 (gr_line (start 82.05600 -74.40000) (end 87.15600 -74.40000) (layer Edge.Cuts) (width 0.2))
 (gr_line (start 96.15600 -74.40000) (end 101.25600 -74.40000) (layer Edge.Cuts) (width 0.2))
 (gr_line (start 87.10600 -117.90000) (end 87.10600 -118.35000) (layer Edge.Cuts) (width 0.2))
 (gr_line (start 87.05600 -118.40000) (end 87.10600 -118.35000) (layer Edge.Cuts) (width 0.2))
 (gr_line (start 88.20600 -117.90000) (end 88.20600 -118.35000) (layer Edge.Cuts) (width 0.2))
 (gr_line (start 88.20600 -118.35000) (end 88.25600 -118.40000) (layer Edge.Cuts) (width 0.2))
 (gr_line (start 83.05600 -88.80000) (end 83.65600 -88.80000) (layer Edge.Cuts) (width 0.2))
 (gr_line (start 99.65600 -88.80000) (end 100.25600 -88.80000) (layer Edge.Cuts) (width 0.2))
 (gr_line (start 95.05600 -118.40000) (end 95.10600 -118.35000) (layer Edge.Cuts) (width 0.2))
 (gr_line (start 95.10600 -117.90000) (end 95.10600 -118.35000) (layer Edge.Cuts) (width 0.2))
 (gr_line (start 96.20600 -118.35000) (end 96.25600 -118.40000) (layer Edge.Cuts) (width 0.2))
 (gr_line (start 96.20600 -117.90000) (end 96.20600 -118.35000) (layer Edge.Cuts) (width 0.2))
 (gr_line (start 99.15600 -118.40000) (end 99.75600 -118.40000) (layer Edge.Cuts) (width 0.2))
 (gr_line (start 91.65600 -118.40000) (end 95.05600 -118.40000) (layer Edge.Cuts) (width 0.2))
 (gr_line (start 96.25600 -118.40000) (end 99.15600 -118.40000) (layer Edge.Cuts) (width 0.2))
 (gr_line (start 100.25600 -88.80000) (end 101.65600 -88.80000) (layer Edge.Cuts) (width 0.2))
 (gr_line (start 81.65600 -112.40000) (end 82.65600 -111.40000) (layer Edge.Cuts) (width 0.2))
 (gr_line (start 82.65600 -105.39999) (end 82.65600 -111.40000) (layer Edge.Cuts) (width 0.2))
 (gr_line (start 81.65600 -104.39999) (end 82.65600 -105.39999) (layer Edge.Cuts) (width 0.2))
 (gr_line (start 81.65600 -103.65000) (end 81.65600 -104.39999) (layer Edge.Cuts) (width 0.2))
 (gr_line (start 81.65600 -112.40000) (end 81.65600 -117.39999) (layer Edge.Cuts) (width 0.2))
 (gr_line (start 101.65600 -112.40000) (end 101.65600 -117.80000) (layer Edge.Cuts) (width 0.2))
 (gr_line (start 101.65600 -103.65000) (end 101.65600 -104.39999) (layer Edge.Cuts) (width 0.2))
 (gr_line (start 100.65600 -105.39999) (end 101.65600 -104.39999) (layer Edge.Cuts) (width 0.2))
 (gr_line (start 100.65600 -105.39999) (end 100.65600 -111.40000) (layer Edge.Cuts) (width 0.2))
 (gr_line (start 100.65600 -111.40000) (end 101.65600 -112.40000) (layer Edge.Cuts) (width 0.2))
 (gr_line (start 83.05600 -96.00000) (end 83.65600 -96.00000) (layer Edge.Cuts) (width 0.2))
 (gr_line (start 81.65600 -96.00000) (end 83.05600 -96.00000) (layer Edge.Cuts) (width 0.2))
 (gr_line (start 81.65600 -96.00000) (end 81.65600 -103.65000) (layer Edge.Cuts) (width 0.2))
 (gr_line (start 101.65600 -96.00000) (end 101.65600 -103.65000) (layer Edge.Cuts) (width 0.2))
 (gr_line (start 100.25600 -96.00000) (end 101.65600 -96.00000) (layer Edge.Cuts) (width 0.2))
 (gr_line (start 99.65600 -96.00000) (end 100.25600 -96.00000) (layer Edge.Cuts) (width 0.2))
 (segment (start 96.73600 -87.51000) (end 97.30600 -86.94000) (width 1.2) (layer B.Cu) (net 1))
 (segment (start 97.30600 -86.94000) (end 99.27600 -86.94000) (width 1.2) (layer B.Cu) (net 1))
 (segment (start 96.73600 -84.97000) (end 97.30600 -84.40000) (width 1.2) (layer B.Cu) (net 1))
 (segment (start 97.30600 -84.40000) (end 99.27600 -84.40000) (width 1.2) (layer B.Cu) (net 1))
 (segment (start 96.73600 -82.40000) (end 97.27600 -81.86000) (width 1.2) (layer B.Cu) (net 1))
 (segment (start 97.27600 -81.86000) (end 99.27600 -81.86000) (width 1.2) (layer B.Cu) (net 1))
 (segment (start 96.73600 -79.89000) (end 97.30600 -79.32000) (width 1.2) (layer B.Cu) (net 1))
 (segment (start 97.30600 -79.32000) (end 99.27600 -79.32000) (width 1.2) (layer B.Cu) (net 1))
 (segment (start 96.73600 -77.35000) (end 97.30600 -76.78000) (width 1.2) (layer B.Cu) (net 1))
 (segment (start 97.30600 -76.78000) (end 99.27600 -76.78000) (width 1.2) (layer B.Cu) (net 1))
 (segment (start 86.00600 -84.40000) (end 86.57600 -84.97000) (width 1.2) (layer B.Cu) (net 1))
 (segment (start 84.03600 -84.40000) (end 86.00600 -84.40000) (width 1.2) (layer B.Cu) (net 1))
 (segment (start 86.00600 -81.86000) (end 86.57600 -82.43000) (width 1.2) (layer B.Cu) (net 1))
 (segment (start 84.03600 -81.86000) (end 86.00600 -81.86000) (width 1.2) (layer B.Cu) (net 1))
 (segment (start 86.00600 -79.32000) (end 86.57600 -79.89000) (width 1.2) (layer B.Cu) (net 1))
 (segment (start 84.03600 -79.32000) (end 86.00600 -79.32000) (width 1.2) (layer B.Cu) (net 1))
 (segment (start 86.00600 -76.78000) (end 86.57600 -77.35000) (width 1.2) (layer B.Cu) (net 1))
 (segment (start 84.03600 -76.78000) (end 86.00600 -76.78000) (width 1.2) (layer B.Cu) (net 1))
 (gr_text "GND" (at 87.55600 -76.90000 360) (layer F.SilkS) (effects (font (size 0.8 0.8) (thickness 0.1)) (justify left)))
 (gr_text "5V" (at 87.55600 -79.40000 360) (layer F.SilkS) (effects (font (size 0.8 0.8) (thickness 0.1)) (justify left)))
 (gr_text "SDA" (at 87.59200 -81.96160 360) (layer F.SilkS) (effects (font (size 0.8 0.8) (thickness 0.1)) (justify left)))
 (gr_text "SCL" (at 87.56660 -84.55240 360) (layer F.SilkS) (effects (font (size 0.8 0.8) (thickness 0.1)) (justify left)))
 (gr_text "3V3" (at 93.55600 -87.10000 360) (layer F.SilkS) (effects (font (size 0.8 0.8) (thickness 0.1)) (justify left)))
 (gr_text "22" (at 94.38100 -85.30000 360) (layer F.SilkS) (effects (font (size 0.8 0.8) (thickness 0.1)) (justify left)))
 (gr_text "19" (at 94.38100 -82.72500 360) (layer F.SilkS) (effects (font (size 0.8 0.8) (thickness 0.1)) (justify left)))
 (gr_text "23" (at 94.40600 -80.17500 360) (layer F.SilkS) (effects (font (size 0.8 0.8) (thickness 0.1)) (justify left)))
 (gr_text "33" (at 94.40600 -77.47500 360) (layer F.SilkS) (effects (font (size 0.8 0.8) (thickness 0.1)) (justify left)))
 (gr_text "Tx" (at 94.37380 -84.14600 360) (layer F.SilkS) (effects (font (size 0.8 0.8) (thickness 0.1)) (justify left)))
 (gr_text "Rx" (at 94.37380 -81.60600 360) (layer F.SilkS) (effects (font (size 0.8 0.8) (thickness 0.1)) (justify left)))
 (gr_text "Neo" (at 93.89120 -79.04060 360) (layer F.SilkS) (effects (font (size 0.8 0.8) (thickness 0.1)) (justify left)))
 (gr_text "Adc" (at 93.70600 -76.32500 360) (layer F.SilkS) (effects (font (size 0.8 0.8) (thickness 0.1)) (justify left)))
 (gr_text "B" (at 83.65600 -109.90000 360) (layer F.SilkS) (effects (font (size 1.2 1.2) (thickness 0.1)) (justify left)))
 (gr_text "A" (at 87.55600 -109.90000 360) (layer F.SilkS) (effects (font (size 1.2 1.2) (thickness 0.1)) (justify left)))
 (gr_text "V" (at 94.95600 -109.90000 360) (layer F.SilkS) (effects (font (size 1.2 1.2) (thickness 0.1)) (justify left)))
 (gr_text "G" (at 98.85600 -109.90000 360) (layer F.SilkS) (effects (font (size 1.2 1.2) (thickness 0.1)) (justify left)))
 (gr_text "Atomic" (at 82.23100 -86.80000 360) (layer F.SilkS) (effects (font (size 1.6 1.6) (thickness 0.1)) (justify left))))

